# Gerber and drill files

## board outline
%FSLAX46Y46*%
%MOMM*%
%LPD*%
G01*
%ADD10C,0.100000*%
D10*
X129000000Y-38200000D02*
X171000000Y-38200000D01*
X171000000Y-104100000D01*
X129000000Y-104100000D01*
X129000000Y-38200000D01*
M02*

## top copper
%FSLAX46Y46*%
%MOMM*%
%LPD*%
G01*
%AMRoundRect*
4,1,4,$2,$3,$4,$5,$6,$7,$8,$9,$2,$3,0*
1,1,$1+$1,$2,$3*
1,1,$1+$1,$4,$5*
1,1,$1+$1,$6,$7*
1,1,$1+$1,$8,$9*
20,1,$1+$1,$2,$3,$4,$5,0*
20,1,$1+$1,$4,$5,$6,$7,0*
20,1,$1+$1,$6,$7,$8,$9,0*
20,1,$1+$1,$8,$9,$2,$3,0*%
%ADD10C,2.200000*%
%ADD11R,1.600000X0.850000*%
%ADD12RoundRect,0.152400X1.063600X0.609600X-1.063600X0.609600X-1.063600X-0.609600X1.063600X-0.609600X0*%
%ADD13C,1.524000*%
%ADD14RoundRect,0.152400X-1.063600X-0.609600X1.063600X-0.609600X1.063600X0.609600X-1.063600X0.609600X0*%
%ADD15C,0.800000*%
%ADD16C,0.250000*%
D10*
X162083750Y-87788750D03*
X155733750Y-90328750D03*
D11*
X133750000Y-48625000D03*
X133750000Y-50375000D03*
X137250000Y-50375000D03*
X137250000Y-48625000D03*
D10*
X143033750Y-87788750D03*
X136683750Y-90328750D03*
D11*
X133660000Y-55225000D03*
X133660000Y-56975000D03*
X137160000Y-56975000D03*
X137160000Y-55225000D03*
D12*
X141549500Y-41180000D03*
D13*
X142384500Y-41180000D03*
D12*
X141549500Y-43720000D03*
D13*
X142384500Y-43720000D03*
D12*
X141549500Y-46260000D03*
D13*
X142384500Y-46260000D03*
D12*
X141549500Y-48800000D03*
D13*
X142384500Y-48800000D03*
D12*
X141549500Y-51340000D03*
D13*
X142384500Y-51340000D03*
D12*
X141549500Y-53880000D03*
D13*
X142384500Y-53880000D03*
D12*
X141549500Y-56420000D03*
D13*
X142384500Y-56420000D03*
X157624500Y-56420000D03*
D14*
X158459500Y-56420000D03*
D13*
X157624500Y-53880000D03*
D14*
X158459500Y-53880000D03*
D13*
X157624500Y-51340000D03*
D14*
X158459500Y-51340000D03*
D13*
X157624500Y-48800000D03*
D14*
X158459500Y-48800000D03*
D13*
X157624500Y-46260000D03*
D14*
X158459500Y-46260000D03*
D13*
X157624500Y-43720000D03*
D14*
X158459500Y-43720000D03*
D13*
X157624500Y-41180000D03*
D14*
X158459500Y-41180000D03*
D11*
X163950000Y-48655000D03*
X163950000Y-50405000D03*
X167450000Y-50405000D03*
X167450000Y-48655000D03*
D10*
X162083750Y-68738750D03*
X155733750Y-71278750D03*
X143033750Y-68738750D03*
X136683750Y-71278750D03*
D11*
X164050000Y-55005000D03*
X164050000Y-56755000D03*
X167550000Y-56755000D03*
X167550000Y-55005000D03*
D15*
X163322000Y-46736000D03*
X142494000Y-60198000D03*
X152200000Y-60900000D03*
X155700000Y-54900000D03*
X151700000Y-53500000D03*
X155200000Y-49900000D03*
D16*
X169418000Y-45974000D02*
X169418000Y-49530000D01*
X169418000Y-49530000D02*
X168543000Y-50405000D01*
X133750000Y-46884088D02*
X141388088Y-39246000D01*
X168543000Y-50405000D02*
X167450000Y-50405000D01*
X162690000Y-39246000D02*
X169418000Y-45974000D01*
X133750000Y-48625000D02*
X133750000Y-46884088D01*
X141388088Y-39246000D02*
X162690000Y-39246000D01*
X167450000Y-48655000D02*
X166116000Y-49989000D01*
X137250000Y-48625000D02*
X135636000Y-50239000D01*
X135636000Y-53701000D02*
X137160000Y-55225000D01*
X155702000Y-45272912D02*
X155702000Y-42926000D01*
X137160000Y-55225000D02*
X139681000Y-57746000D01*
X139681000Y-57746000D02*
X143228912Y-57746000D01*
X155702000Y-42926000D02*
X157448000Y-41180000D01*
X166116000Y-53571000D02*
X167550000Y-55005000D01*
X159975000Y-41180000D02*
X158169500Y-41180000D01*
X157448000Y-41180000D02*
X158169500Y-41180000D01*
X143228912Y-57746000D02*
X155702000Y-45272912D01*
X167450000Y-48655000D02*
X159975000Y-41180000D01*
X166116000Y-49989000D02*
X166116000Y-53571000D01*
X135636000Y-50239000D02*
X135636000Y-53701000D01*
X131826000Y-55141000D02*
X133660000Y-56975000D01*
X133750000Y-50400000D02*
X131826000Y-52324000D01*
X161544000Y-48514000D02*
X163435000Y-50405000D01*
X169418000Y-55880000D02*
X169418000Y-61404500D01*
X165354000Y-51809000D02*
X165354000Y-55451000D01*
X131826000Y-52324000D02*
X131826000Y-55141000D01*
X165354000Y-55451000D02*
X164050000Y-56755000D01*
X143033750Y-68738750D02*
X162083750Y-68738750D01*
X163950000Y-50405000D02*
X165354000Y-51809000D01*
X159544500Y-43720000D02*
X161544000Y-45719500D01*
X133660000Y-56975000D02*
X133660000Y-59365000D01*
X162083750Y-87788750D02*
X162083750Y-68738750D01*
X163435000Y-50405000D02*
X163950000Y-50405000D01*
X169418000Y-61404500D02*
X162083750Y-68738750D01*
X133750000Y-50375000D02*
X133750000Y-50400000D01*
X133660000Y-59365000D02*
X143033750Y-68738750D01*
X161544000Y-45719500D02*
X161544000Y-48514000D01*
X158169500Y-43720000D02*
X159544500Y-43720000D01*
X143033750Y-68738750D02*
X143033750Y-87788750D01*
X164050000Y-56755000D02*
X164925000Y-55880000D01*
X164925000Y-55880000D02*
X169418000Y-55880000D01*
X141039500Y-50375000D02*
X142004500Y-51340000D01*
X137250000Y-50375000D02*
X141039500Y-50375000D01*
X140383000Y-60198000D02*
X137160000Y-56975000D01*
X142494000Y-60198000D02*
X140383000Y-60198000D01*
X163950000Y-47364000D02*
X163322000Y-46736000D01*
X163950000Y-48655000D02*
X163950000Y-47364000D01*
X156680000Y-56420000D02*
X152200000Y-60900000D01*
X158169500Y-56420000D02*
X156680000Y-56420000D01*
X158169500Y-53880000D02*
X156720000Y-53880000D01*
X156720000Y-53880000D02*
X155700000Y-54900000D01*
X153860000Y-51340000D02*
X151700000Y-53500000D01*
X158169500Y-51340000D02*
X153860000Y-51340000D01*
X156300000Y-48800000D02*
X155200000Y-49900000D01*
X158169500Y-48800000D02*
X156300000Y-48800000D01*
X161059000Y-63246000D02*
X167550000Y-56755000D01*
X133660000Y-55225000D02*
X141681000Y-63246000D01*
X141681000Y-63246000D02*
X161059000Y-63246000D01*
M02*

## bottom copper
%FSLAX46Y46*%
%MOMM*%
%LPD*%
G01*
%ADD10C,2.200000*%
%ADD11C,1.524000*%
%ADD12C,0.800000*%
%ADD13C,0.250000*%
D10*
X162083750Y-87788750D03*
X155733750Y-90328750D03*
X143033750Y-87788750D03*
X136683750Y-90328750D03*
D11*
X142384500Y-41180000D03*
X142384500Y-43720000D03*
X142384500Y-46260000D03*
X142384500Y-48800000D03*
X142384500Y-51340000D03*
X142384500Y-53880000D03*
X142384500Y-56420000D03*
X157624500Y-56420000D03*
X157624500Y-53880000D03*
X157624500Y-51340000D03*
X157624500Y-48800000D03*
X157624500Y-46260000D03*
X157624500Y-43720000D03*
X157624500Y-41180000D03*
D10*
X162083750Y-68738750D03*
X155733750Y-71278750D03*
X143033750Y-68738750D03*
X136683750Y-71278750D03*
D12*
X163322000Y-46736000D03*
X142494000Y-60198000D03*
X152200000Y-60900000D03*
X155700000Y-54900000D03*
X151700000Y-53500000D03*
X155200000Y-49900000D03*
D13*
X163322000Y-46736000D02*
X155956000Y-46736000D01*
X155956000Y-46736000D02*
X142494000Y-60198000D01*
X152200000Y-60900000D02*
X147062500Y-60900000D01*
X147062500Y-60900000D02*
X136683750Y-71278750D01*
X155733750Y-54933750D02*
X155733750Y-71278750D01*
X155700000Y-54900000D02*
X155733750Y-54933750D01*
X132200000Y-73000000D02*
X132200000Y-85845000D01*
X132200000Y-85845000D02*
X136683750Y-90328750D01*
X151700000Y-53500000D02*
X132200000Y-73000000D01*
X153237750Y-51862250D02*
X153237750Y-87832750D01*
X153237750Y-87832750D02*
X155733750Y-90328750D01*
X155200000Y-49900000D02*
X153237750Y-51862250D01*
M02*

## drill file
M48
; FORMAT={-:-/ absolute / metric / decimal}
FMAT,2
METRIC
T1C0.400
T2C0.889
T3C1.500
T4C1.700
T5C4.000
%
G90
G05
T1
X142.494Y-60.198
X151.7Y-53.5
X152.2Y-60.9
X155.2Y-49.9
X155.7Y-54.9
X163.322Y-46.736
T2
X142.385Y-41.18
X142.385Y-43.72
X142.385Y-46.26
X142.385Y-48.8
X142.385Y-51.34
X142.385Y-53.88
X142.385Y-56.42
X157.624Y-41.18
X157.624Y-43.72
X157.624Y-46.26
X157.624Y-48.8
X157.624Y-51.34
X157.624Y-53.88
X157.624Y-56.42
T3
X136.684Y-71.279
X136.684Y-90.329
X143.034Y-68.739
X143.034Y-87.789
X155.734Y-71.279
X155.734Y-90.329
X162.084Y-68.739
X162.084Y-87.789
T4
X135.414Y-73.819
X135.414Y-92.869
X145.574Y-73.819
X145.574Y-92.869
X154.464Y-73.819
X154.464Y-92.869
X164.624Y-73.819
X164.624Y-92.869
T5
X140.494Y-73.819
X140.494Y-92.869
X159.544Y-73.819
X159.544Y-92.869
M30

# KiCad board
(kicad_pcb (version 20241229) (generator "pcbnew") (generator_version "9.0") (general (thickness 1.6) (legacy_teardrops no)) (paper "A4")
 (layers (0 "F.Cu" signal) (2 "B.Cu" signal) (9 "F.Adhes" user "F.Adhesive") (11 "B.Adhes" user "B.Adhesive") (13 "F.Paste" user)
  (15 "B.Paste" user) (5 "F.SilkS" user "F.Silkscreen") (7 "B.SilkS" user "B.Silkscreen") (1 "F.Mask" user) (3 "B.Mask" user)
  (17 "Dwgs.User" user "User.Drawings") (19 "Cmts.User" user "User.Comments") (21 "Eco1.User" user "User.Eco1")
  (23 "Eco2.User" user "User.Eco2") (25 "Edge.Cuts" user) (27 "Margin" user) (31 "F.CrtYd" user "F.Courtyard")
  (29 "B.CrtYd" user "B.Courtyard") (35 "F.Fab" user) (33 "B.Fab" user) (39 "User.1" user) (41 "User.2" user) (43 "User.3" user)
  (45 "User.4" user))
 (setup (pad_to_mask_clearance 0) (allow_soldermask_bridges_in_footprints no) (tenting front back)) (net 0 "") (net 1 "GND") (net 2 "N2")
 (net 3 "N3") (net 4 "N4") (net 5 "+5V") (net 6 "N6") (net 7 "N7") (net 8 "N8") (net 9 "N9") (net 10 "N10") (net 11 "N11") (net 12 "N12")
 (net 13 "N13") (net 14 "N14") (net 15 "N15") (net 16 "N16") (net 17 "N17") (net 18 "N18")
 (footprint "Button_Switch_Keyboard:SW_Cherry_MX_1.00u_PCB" (layer "F.Cu") (at 162.08375 87.78875)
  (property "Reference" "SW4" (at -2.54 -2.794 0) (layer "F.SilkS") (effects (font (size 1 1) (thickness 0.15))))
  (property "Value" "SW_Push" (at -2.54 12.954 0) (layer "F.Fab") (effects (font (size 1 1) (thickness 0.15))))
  (pad "" np_thru_hole circle (at -7.62 5.08) (size 1.7 1.7) (drill 1.7) (layers "*.Cu" "*.Mask"))
  (pad "" np_thru_hole circle (at -2.54 5.08) (size 4 4) (drill 4) (layers "*.Cu" "*.Mask"))
  (pad "" np_thru_hole circle (at 2.54 5.08) (size 1.7 1.7) (drill 1.7) (layers "*.Cu" "*.Mask"))
  (pad "1" thru_hole circle (at 0 0) (size 2.2 2.2) (drill 1.5) (layers "*.Cu" "*.Mask") (remove_unused_layers no) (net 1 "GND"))
  (pad "2" thru_hole circle (at -6.35 2.54) (size 2.2 2.2) (drill 1.5) (layers "*.Cu" "*.Mask") (remove_unused_layers no) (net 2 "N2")))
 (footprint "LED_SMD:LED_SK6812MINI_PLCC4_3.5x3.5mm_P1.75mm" (layer "F.Cu") (at 135.5 49.5)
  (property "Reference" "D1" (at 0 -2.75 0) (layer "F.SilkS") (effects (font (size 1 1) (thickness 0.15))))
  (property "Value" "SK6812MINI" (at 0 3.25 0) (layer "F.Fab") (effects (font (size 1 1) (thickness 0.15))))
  (pad "1" smd rect (at -1.75 -0.875) (size 1.6 0.85) (layers "F.Cu" "F.Mask" "F.Paste") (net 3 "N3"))
  (pad "2" smd rect (at -1.75 0.875) (size 1.6 0.85) (layers "F.Cu" "F.Mask" "F.Paste") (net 1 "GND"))
  (pad "3" smd rect (at 1.75 0.875) (size 1.6 0.85) (layers "F.Cu" "F.Mask" "F.Paste") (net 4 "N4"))
  (pad "4" smd rect (at 1.75 -0.875) (size 1.6 0.85) (layers "F.Cu" "F.Mask" "F.Paste") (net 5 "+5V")))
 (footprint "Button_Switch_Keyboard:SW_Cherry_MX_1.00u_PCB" (layer "F.Cu") (at 143.03375 87.78875)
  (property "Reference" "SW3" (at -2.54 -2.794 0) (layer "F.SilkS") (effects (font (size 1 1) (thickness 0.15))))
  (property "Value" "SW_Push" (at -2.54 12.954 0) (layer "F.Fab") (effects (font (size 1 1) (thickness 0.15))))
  (pad "" np_thru_hole circle (at -7.62 5.08) (size 1.7 1.7) (drill 1.7) (layers "*.Cu" "*.Mask"))
  (pad "" np_thru_hole circle (at -2.54 5.08) (size 4 4) (drill 4) (layers "*.Cu" "*.Mask"))
  (pad "" np_thru_hole circle (at 2.54 5.08) (size 1.7 1.7) (drill 1.7) (layers "*.Cu" "*.Mask"))
  (pad "1" thru_hole circle (at 0 0) (size 2.2 2.2) (drill 1.5) (layers "*.Cu" "*.Mask") (remove_unused_layers no) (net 1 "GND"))
  (pad "2" thru_hole circle (at -6.35 2.54) (size 2.2 2.2) (drill 1.5) (layers "*.Cu" "*.Mask") (remove_unused_layers no) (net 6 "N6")))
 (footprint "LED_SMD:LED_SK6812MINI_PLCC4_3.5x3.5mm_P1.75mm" (layer "F.Cu") (at 135.41 56.1)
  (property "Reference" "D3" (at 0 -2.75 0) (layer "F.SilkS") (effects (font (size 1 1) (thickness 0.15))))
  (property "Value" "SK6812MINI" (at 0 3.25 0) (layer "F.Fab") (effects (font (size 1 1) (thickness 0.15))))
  (pad "1" smd rect (at -1.75 -0.875) (size 1.6 0.85) (layers "F.Cu" "F.Mask" "F.Paste") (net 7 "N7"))
  (pad "2" smd rect (at -1.75 0.875) (size 1.6 0.85) (layers "F.Cu" "F.Mask" "F.Paste") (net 1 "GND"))
  (pad "3" smd rect (at 1.75 0.875) (size 1.6 0.85) (layers "F.Cu" "F.Mask" "F.Paste") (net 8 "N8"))
  (pad "4" smd rect (at 1.75 -0.875) (size 1.6 0.85) (layers "F.Cu" "F.Mask" "F.Paste") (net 5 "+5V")))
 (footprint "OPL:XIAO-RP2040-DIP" (layer "F.Cu") (at 150.0045 48.8)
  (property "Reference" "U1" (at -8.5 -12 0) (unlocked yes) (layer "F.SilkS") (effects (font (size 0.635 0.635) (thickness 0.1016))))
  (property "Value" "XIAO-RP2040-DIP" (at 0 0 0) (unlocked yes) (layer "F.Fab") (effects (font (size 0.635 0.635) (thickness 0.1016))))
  (pad "1" smd roundrect (at -8.455 -7.62 180) (size 2.432 1.524) (layers "F.Cu" "F.Mask") (roundrect_rratio 0.1) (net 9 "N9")
   (thermal_bridge_angle 45))
  (pad "1" thru_hole circle (at -7.62 -7.62 180) (size 1.524 1.524) (drill 0.889) (layers "*.Cu" "*.Mask") (remove_unused_layers no)
   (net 9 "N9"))
  (pad "2" smd roundrect (at -8.455 -5.08 180) (size 2.432 1.524) (layers "F.Cu" "F.Mask") (roundrect_rratio 0.1) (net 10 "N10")
   (thermal_bridge_angle 45))
  (pad "2" thru_hole circle (at -7.62 -5.08 180) (size 1.524 1.524) (drill 0.889) (layers "*.Cu" "*.Mask") (remove_unused_layers no)
   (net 10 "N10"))
  (pad "3" smd roundrect (at -8.455 -2.54 180) (size 2.432 1.524) (layers "F.Cu" "F.Mask") (roundrect_rratio 0.1) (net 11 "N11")
   (thermal_bridge_angle 45))
  (pad "3" thru_hole circle (at -7.62 -2.54 180) (size 1.524 1.524) (drill 0.889) (layers "*.Cu" "*.Mask") (remove_unused_layers no)
   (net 11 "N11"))
  (pad "4" smd roundrect (at -8.455 0 180) (size 2.432 1.524) (layers "F.Cu" "F.Mask") (roundrect_rratio 0.1) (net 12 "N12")
   (thermal_bridge_angle 45))
  (pad "4" thru_hole circle (at -7.62 0 180) (size 1.524 1.524) (drill 0.889) (layers "*.Cu" "*.Mask") (remove_unused_layers no)
   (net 12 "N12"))
  (pad "5" smd roundrect (at -8.455 2.54 180) (size 2.432 1.524) (layers "F.Cu" "F.Mask") (roundrect_rratio 0.1) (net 4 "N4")
   (thermal_bridge_angle 45))
  (pad "5" thru_hole circle (at -7.62 2.54 180) (size 1.524 1.524) (drill 0.889) (layers "*.Cu" "*.Mask") (remove_unused_layers no)
   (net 4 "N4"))
  (pad "6" smd roundrect (at -8.455 5.08 180) (size 2.432 1.524) (layers "F.Cu" "F.Mask") (roundrect_rratio 0.1) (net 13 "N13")
   (thermal_bridge_angle 45))
  (pad "6" thru_hole circle (at -7.62 5.08 180) (size 1.524 1.524) (drill 0.889) (layers "*.Cu" "*.Mask") (remove_unused_layers no)
   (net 13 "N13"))
  (pad "7" smd roundrect (at -8.455 7.62 180) (size 2.432 1.524) (layers "F.Cu" "F.Mask") (roundrect_rratio 0.1) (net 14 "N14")
   (thermal_bridge_angle 45))
  (pad "7" thru_hole circle (at -7.62 7.62 180) (size 1.524 1.524) (drill 0.889) (layers "*.Cu" "*.Mask") (remove_unused_layers no)
   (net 14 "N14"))
  (pad "8" thru_hole circle (at 7.62 7.62) (size 1.524 1.524) (drill 0.889) (layers "*.Cu" "*.Mask") (remove_unused_layers no)
   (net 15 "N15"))
  (pad "8" smd roundrect (at 8.455 7.62) (size 2.432 1.524) (layers "F.Cu" "F.Mask") (roundrect_rratio 0.1) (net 15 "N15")
   (thermal_bridge_angle 45))
  (pad "9" thru_hole circle (at 7.62 5.08) (size 1.524 1.524) (drill 0.889) (layers "*.Cu" "*.Mask") (remove_unused_layers no)
   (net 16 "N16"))
  (pad "9" smd roundrect (at 8.455 5.08) (size 2.432 1.524) (layers "F.Cu" "F.Mask") (roundrect_rratio 0.1) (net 16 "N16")
   (thermal_bridge_angle 45))
  (pad "10" thru_hole circle (at 7.62 2.54) (size 1.524 1.524) (drill 0.889) (layers "*.Cu" "*.Mask") (remove_unused_layers no) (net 6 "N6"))
  (pad "10" smd roundrect (at 8.455 2.54) (size 2.432 1.524) (layers "F.Cu" "F.Mask") (roundrect_rratio 0.1) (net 6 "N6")
   (thermal_bridge_angle 45))
  (pad "11" thru_hole circle (at 7.62 0) (size 1.524 1.524) (drill 0.889) (layers "*.Cu" "*.Mask") (remove_unused_layers no) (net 2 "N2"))
  (pad "11" smd roundrect (at 8.455 0) (size 2.432 1.524) (layers "F.Cu" "F.Mask") (roundrect_rratio 0.1) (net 2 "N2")
   (thermal_bridge_angle 45))
  (pad "12" thru_hole circle (at 7.62 -2.54) (size 1.524 1.524) (drill 0.889) (layers "*.Cu" "*.Mask") (remove_unused_layers no)
   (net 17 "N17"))
  (pad "12" smd roundrect (at 8.455 -2.54) (size 2.432 1.524) (layers "F.Cu" "F.Mask") (roundrect_rratio 0.1) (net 17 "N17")
   (thermal_bridge_angle 45))
  (pad "13" thru_hole circle (at 7.62 -5.08) (size 1.524 1.524) (drill 0.889) (layers "*.Cu" "*.Mask") (remove_unused_layers no)
   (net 1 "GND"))
  (pad "13" smd roundrect (at 8.455 -5.08) (size 2.432 1.524) (layers "F.Cu" "F.Mask") (roundrect_rratio 0.1) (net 1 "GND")
   (thermal_bridge_angle 45))
  (pad "14" thru_hole circle (at 7.62 -7.62) (size 1.524 1.524) (drill 0.889) (layers "*.Cu" "*.Mask") (remove_unused_layers no)
   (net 5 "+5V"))
  (pad "14" smd roundrect (at 8.455 -7.62) (size 2.432 1.524) (layers "F.Cu" "F.Mask") (roundrect_rratio 0.1) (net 5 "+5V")
   (thermal_bridge_angle 45)))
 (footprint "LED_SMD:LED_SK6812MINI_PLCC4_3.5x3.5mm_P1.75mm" (layer "F.Cu") (at 165.7 49.53)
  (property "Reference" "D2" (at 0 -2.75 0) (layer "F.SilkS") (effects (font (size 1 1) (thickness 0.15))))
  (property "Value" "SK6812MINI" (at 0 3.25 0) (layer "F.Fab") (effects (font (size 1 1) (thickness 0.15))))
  (pad "1" smd rect (at -1.75 -0.875) (size 1.6 0.85) (layers "F.Cu" "F.Mask" "F.Paste") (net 8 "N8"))
  (pad "2" smd rect (at -1.75 0.875) (size 1.6 0.85) (layers "F.Cu" "F.Mask" "F.Paste") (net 1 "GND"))
  (pad "3" smd rect (at 1.75 0.875) (size 1.6 0.85) (layers "F.Cu" "F.Mask" "F.Paste") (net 3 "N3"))
  (pad "4" smd rect (at 1.75 -0.875) (size 1.6 0.85) (layers "F.Cu" "F.Mask" "F.Paste") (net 5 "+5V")))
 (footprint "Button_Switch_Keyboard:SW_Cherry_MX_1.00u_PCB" (layer "F.Cu") (at 162.08375 68.73875)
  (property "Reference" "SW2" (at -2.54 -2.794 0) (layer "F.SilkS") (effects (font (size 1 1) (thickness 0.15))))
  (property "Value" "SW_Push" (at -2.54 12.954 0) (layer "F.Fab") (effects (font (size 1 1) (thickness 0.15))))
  (pad "" np_thru_hole circle (at -7.62 5.08) (size 1.7 1.7) (drill 1.7) (layers "*.Cu" "*.Mask"))
  (pad "" np_thru_hole circle (at -2.54 5.08) (size 4 4) (drill 4) (layers "*.Cu" "*.Mask"))
  (pad "" np_thru_hole circle (at 2.54 5.08) (size 1.7 1.7) (drill 1.7) (layers "*.Cu" "*.Mask"))
  (pad "1" thru_hole circle (at 0 0) (size 2.2 2.2) (drill 1.5) (layers "*.Cu" "*.Mask") (remove_unused_layers no) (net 1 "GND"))
  (pad "2" thru_hole circle (at -6.35 2.54) (size 2.2 2.2) (drill 1.5) (layers "*.Cu" "*.Mask") (remove_unused_layers no) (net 16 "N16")))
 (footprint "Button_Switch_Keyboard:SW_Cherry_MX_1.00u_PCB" (layer "F.Cu") (at 143.03375 68.73875)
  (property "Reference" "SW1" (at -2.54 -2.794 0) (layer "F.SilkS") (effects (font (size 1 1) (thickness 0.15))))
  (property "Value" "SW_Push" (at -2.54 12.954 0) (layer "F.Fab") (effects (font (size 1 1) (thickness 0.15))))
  (pad "" np_thru_hole circle (at -7.62 5.08) (size 1.7 1.7) (drill 1.7) (layers "*.Cu" "*.Mask"))
  (pad "" np_thru_hole circle (at -2.54 5.08) (size 4 4) (drill 4) (layers "*.Cu" "*.Mask"))
  (pad "" np_thru_hole circle (at 2.54 5.08) (size 1.7 1.7) (drill 1.7) (layers "*.Cu" "*.Mask"))
  (pad "1" thru_hole circle (at 0 0) (size 2.2 2.2) (drill 1.5) (layers "*.Cu" "*.Mask") (remove_unused_layers no) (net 1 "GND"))
  (pad "2" thru_hole circle (at -6.35 2.54) (size 2.2 2.2) (drill 1.5) (layers "*.Cu" "*.Mask") (remove_unused_layers no) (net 15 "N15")))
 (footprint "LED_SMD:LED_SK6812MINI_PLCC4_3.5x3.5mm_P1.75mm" (layer "F.Cu") (at 165.8 55.88)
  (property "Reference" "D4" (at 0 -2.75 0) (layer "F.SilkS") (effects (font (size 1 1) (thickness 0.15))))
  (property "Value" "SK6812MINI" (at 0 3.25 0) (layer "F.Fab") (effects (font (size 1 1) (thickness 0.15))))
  (pad "1" smd rect (at -1.75 -0.875) (size 1.6 0.85) (layers "F.Cu" "F.Mask" "F.Paste") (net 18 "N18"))
  (pad "2" smd rect (at -1.75 0.875) (size 1.6 0.85) (layers "F.Cu" "F.Mask" "F.Paste") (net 1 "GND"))
  (pad "3" smd rect (at 1.75 0.875) (size 1.6 0.85) (layers "F.Cu" "F.Mask" "F.Paste") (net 7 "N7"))
  (pad "4" smd rect (at 1.75 -0.875) (size 1.6 0.85) (layers "F.Cu" "F.Mask" "F.Paste") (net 5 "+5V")))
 (gr_rect (start 129 38.2) (end 171 104.1) (stroke (width 0.1) (type default)) (fill no) (layer "Edge.Cuts"))
 (segment (start 169.418 45.974) (end 169.418 49.53) (width 0.25) (layer "F.Cu") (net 3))
 (segment (start 169.418 49.53) (end 168.543 50.405) (width 0.25) (layer "F.Cu") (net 3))
 (segment (start 133.75 46.884088) (end 141.388088 39.246) (width 0.25) (layer "F.Cu") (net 3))
 (segment (start 168.543 50.405) (end 167.45 50.405) (width 0.25) (layer "F.Cu") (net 3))
 (segment (start 162.69 39.246) (end 169.418 45.974) (width 0.25) (layer "F.Cu") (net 3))
 (segment (start 133.75 48.625) (end 133.75 46.884088) (width 0.25) (layer "F.Cu") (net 3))
 (segment (start 141.388088 39.246) (end 162.69 39.246) (width 0.25) (layer "F.Cu") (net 3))
 (segment (start 167.45 48.655) (end 166.116 49.989) (width 0.25) (layer "F.Cu") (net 5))
 (segment (start 137.25 48.625) (end 135.636 50.239) (width 0.25) (layer "F.Cu") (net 5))
 (segment (start 135.636 53.701) (end 137.16 55.225) (width 0.25) (layer "F.Cu") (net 5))
 (segment (start 155.702 45.272912) (end 155.702 42.926) (width 0.25) (layer "F.Cu") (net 5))
 (segment (start 137.16 55.225) (end 139.681 57.746) (width 0.25) (layer "F.Cu") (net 5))
 (segment (start 139.681 57.746) (end 143.228912 57.746) (width 0.25) (layer "F.Cu") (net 5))
 (segment (start 155.702 42.926) (end 157.448 41.18) (width 0.25) (layer "F.Cu") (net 5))
 (segment (start 166.116 53.571) (end 167.55 55.005) (width 0.25) (layer "F.Cu") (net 5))
 (segment (start 159.975 41.18) (end 158.1695 41.18) (width 0.25) (layer "F.Cu") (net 5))
 (segment (start 157.448 41.18) (end 158.1695 41.18) (width 0.25) (layer "F.Cu") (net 5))
 (segment (start 143.228912 57.746) (end 155.702 45.272912) (width 0.25) (layer "F.Cu") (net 5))
 (segment (start 167.45 48.655) (end 159.975 41.18) (width 0.25) (layer "F.Cu") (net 5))
 (segment (start 166.116 49.989) (end 166.116 53.571) (width 0.25) (layer "F.Cu") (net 5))
 (segment (start 135.636 50.239) (end 135.636 53.701) (width 0.25) (layer "F.Cu") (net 5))
 (segment (start 131.826 55.141) (end 133.66 56.975) (width 0.25) (layer "F.Cu") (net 1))
 (segment (start 133.75 50.4) (end 131.826 52.324) (width 0.25) (layer "F.Cu") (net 1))
 (segment (start 161.544 48.514) (end 163.435 50.405) (width 0.25) (layer "F.Cu") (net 1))
 (segment (start 169.418 55.88) (end 169.418 61.4045) (width 0.25) (layer "F.Cu") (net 1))
 (segment (start 165.354 51.809) (end 165.354 55.451) (width 0.25) (layer "F.Cu") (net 1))
 (segment (start 131.826 52.324) (end 131.826 55.141) (width 0.25) (layer "F.Cu") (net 1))
 (segment (start 165.354 55.451) (end 164.05 56.755) (width 0.25) (layer "F.Cu") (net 1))
 (segment (start 143.03375 68.73875) (end 162.08375 68.73875) (width 0.25) (layer "F.Cu") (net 1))
 (segment (start 163.95 50.405) (end 165.354 51.809) (width 0.25) (layer "F.Cu") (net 1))
 (segment (start 159.5445 43.72) (end 161.544 45.7195) (width 0.25) (layer "F.Cu") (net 1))
 (segment (start 133.66 56.975) (end 133.66 59.365) (width 0.25) (layer "F.Cu") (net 1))
 (segment (start 162.08375 87.78875) (end 162.08375 68.73875) (width 0.25) (layer "F.Cu") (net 1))
 (segment (start 163.435 50.405) (end 163.95 50.405) (width 0.25) (layer "F.Cu") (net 1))
 (segment (start 169.418 61.4045) (end 162.08375 68.73875) (width 0.25) (layer "F.Cu") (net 1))
 (segment (start 133.75 50.375) (end 133.75 50.4) (width 0.25) (layer "F.Cu") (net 1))
 (segment (start 133.66 59.365) (end 143.03375 68.73875) (width 0.25) (layer "F.Cu") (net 1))
 (segment (start 161.544 45.7195) (end 161.544 48.514) (width 0.25) (layer "F.Cu") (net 1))
 (segment (start 158.1695 43.72) (end 159.5445 43.72) (width 0.25) (layer "F.Cu") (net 1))
 (segment (start 143.03375 68.73875) (end 143.03375 87.78875) (width 0.25) (layer "F.Cu") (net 1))
 (segment (start 164.05 56.755) (end 164.925 55.88) (width 0.25) (layer "F.Cu") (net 1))
 (segment (start 164.925 55.88) (end 169.418 55.88) (width 0.25) (layer "F.Cu") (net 1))
 (segment (start 141.0395 50.375) (end 142.0045 51.34) (width 0.25) (layer "F.Cu") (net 4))
 (segment (start 137.25 50.375) (end 141.0395 50.375) (width 0.25) (layer "F.Cu") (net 4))
 (segment (start 140.383 60.198) (end 137.16 56.975) (width 0.25) (layer "F.Cu") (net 8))
 (segment (start 142.494 60.198) (end 140.383 60.198) (width 0.25) (layer "F.Cu") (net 8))
 (segment (start 163.95 47.364) (end 163.322 46.736) (width 0.25) (layer "F.Cu") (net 8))
 (segment (start 163.95 48.655) (end 163.95 47.364) (width 0.25) (layer "F.Cu") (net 8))
 (via (at 163.322 46.736) (size 0.8) (drill 0.4) (layers "F.Cu" "B.Cu") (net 8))
 (via (at 142.494 60.198) (size 0.8) (drill 0.4) (layers "F.Cu" "B.Cu") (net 8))
 (segment (start 163.322 46.736) (end 155.956 46.736) (width 0.25) (layer "B.Cu") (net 8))
 (segment (start 155.956 46.736) (end 142.494 60.198) (width 0.25) (layer "B.Cu") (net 8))
 (segment (start 156.68 56.42) (end 152.2 60.9) (width 0.25) (layer "F.Cu") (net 15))
 (segment (start 158.1695 56.42) (end 156.68 56.42) (width 0.25) (layer "F.Cu") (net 15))
 (via (at 152.2 60.9) (size 0.8) (drill 0.4) (layers "F.Cu" "B.Cu") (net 15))
 (segment (start 152.2 60.9) (end 147.0625 60.9) (width 0.25) (layer "B.Cu") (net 15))
 (segment (start 147.0625 60.9) (end 136.68375 71.27875) (width 0.25) (layer "B.Cu") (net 15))
 (segment (start 158.1695 53.88) (end 156.72 53.88) (width 0.25) (layer "F.Cu") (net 16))
 (segment (start 156.72 53.88) (end 155.7 54.9) (width 0.25) (layer "F.Cu") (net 16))
 (via (at 155.7 54.9) (size 0.8) (drill 0.4) (layers "F.Cu" "B.Cu") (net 16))
 (segment (start 155.73375 54.93375) (end 155.73375 71.27875) (width 0.25) (layer "B.Cu") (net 16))
 (segment (start 155.7 54.9) (end 155.73375 54.93375) (width 0.25) (layer "B.Cu") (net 16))
 (segment (start 153.86 51.34) (end 151.7 53.5) (width 0.25) (layer "F.Cu") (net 6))
 (segment (start 158.1695 51.34) (end 153.86 51.34) (width 0.25) (layer "F.Cu") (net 6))
 (via (at 151.7 53.5) (size 0.8) (drill 0.4) (layers "F.Cu" "B.Cu") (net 6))
 (segment (start 132.2 73) (end 132.2 85.845) (width 0.25) (layer "B.Cu") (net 6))
 (segment (start 132.2 85.845) (end 136.68375 90.32875) (width 0.25) (layer "B.Cu") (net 6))
 (segment (start 151.7 53.5) (end 132.2 73) (width 0.25) (layer "B.Cu") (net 6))
 (segment (start 156.3 48.8) (end 155.2 49.9) (width 0.25) (layer "F.Cu") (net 2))
 (segment (start 158.1695 48.8) (end 156.3 48.8) (width 0.25) (layer "F.Cu") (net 2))
 (via (at 155.2 49.9) (size 0.8) (drill 0.4) (layers "F.Cu" "B.Cu") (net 2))
 (segment (start 153.23775 51.86225) (end 153.23775 87.83275) (width 0.25) (layer "B.Cu") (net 2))
 (segment (start 153.23775 87.83275) (end 155.73375 90.32875) (width 0.25) (layer "B.Cu") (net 2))
 (segment (start 155.2 49.9) (end 153.23775 51.86225) (width 0.25) (layer "B.Cu") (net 2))
 (segment (start 161.059 63.246) (end 167.55 56.755) (width 0.25) (layer "F.Cu") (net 7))
 (segment (start 133.66 55.225) (end 141.681 63.246) (width 0.25) (layer "F.Cu") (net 7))
 (segment (start 141.681 63.246) (end 161.059 63.246) (width 0.25) (layer "F.Cu") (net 7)))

